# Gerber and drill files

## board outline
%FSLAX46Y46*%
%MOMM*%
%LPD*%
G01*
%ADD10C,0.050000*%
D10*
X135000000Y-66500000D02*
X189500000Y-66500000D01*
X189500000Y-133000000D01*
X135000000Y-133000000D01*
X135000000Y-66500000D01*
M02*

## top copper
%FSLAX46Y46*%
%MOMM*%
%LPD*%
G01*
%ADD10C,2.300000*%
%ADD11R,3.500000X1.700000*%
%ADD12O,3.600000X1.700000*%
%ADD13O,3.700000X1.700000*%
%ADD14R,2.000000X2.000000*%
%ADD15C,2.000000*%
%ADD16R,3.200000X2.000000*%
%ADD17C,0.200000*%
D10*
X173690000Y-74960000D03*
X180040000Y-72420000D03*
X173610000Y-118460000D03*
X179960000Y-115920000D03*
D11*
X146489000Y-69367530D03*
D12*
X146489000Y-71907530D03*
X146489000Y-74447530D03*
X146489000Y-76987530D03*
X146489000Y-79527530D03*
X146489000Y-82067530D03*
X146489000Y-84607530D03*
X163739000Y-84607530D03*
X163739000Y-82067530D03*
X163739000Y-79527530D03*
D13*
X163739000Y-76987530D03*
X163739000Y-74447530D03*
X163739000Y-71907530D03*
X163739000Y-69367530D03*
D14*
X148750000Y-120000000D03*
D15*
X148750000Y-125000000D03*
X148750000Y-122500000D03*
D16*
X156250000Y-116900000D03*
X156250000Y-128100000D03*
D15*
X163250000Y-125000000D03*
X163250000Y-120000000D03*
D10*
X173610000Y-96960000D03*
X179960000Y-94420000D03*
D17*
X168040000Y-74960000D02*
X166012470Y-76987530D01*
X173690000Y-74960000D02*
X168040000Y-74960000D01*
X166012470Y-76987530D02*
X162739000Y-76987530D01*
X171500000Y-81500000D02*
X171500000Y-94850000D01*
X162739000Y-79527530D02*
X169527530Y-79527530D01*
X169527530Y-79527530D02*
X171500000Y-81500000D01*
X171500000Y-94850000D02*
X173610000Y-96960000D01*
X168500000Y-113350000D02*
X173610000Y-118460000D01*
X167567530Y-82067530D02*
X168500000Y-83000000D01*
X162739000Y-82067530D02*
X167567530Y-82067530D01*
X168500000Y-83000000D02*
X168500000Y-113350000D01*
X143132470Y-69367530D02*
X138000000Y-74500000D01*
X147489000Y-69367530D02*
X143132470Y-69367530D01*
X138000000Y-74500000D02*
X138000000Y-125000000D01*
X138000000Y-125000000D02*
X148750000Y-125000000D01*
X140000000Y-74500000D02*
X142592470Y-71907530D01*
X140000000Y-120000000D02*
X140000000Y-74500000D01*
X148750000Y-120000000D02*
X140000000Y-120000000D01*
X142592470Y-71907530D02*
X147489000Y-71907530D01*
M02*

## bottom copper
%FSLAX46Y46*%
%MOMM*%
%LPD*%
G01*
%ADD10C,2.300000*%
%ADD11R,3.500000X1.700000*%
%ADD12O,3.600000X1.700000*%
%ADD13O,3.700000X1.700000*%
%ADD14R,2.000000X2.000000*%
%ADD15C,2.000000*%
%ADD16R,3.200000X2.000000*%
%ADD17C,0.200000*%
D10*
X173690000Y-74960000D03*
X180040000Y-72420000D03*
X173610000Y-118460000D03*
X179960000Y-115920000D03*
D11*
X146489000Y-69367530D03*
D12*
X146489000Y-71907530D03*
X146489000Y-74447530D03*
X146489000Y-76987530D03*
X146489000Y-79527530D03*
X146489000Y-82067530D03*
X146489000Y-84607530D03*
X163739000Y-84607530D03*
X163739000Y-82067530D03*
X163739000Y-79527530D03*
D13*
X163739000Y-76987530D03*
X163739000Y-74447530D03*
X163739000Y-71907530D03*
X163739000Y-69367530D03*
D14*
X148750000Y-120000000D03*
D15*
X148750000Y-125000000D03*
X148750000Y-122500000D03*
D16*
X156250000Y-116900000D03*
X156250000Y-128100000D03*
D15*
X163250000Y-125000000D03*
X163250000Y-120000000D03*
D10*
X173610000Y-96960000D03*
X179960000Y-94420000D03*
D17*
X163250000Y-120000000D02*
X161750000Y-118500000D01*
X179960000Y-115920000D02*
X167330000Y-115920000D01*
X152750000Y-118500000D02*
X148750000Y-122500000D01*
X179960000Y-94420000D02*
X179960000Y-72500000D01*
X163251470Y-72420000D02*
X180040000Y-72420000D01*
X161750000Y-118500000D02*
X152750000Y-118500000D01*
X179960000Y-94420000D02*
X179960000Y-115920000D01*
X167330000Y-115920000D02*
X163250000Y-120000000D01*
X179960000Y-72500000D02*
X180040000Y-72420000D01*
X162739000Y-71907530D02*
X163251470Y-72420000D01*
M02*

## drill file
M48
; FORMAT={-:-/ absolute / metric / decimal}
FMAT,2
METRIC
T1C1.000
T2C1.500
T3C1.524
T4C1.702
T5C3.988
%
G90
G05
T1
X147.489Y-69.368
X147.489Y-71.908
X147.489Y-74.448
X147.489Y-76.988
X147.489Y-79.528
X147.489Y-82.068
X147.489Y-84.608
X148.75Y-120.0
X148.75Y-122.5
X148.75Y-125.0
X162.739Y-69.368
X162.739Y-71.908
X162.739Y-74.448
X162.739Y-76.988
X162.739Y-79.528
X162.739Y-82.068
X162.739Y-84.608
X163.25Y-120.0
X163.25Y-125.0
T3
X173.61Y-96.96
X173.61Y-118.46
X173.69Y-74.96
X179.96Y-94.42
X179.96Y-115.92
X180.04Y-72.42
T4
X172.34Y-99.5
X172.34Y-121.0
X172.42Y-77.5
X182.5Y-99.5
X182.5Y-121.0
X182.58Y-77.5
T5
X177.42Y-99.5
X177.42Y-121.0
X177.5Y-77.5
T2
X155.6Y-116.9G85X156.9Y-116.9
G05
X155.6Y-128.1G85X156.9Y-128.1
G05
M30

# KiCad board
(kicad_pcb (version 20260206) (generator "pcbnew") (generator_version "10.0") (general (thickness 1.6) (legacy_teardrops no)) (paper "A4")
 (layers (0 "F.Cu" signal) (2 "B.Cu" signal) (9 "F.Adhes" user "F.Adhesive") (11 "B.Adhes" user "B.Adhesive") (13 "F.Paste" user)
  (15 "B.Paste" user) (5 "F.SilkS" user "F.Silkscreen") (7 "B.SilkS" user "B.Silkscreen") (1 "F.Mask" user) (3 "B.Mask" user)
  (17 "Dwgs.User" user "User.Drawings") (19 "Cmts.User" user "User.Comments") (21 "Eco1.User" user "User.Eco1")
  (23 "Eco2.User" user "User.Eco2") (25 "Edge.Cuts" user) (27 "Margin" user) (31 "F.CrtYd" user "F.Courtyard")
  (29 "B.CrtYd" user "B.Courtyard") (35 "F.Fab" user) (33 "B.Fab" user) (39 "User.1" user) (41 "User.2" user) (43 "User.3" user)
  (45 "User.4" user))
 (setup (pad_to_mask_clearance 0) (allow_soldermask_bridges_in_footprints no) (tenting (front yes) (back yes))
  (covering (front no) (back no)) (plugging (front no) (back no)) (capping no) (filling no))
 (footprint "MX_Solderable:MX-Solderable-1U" (layer "F.Cu") (at 177.5 77.5)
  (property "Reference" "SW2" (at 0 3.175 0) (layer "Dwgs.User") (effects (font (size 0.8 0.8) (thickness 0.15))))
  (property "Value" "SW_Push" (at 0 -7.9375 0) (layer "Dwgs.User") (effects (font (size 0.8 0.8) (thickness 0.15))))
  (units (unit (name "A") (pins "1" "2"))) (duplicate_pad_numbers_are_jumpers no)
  (pad "" np_thru_hole circle (at -5.08 0 48.099) (size 1.7018 1.7018) (drill 1.7018) (layers "*.Cu" "*.Mask"))
  (pad "" np_thru_hole circle (at 0 0) (size 3.9878 3.9878) (drill 3.9878) (layers "*.Cu" "*.Mask"))
  (pad "" np_thru_hole circle (at 5.08 0 48.099) (size 1.7018 1.7018) (drill 1.7018) (layers "*.Cu" "*.Mask"))
  (pad "1" thru_hole circle (at -3.81 -2.54) (size 2.3 2.3) (drill 1.524) (layers "*.Cu" "B.Mask") (remove_unused_layers no)
   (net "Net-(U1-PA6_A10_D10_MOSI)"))
  (pad "2" thru_hole circle (at 2.54 -5.08) (size 2.3 2.3) (drill 1.524) (layers "*.Cu" "B.Mask") (remove_unused_layers no)
   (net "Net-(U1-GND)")))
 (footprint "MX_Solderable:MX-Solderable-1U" (layer "F.Cu") (at 177.42 121)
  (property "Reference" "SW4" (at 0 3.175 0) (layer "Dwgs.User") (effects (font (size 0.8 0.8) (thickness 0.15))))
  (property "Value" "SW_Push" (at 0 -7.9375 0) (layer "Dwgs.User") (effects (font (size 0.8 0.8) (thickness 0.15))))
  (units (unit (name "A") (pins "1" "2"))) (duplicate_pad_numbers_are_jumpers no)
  (pad "" np_thru_hole circle (at -5.08 0 48.099) (size 1.7018 1.7018) (drill 1.7018) (layers "*.Cu" "*.Mask"))
  (pad "" np_thru_hole circle (at 0 0) (size 3.9878 3.9878) (drill 3.9878) (layers "*.Cu" "*.Mask"))
  (pad "" np_thru_hole circle (at 5.08 0 48.099) (size 1.7018 1.7018) (drill 1.7018) (layers "*.Cu" "*.Mask"))
  (pad "1" thru_hole circle (at -3.81 -2.54) (size 2.3 2.3) (drill 1.524) (layers "*.Cu" "B.Mask") (remove_unused_layers no)
   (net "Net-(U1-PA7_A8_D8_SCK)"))
  (pad "2" thru_hole circle (at 2.54 -5.08) (size 2.3 2.3) (drill 1.524) (layers "*.Cu" "B.Mask") (remove_unused_layers no)
   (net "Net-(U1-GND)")))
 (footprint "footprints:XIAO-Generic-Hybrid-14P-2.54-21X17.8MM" (layer "F.Cu") (at 155.114 76.98753)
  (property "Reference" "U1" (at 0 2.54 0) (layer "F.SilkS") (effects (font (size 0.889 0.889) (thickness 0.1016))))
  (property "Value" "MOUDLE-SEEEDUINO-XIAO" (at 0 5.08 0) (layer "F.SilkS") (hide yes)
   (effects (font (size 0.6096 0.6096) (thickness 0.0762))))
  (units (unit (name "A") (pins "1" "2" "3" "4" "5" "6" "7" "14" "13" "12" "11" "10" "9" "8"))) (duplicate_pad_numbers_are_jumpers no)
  (pad "1" thru_hole rect (at -7.625 -7.62) (size 3.5 1.7) (drill 1 (offset -1 0)) (layers "*.Cu" "*.Mask") (remove_unused_layers no)
   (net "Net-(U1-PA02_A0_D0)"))
  (pad "2" thru_hole oval (at -7.625 -5.08) (size 3.6 1.7) (drill 1 (offset -1 0)) (layers "*.Cu" "*.Mask") (remove_unused_layers no)
   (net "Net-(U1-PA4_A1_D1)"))
  (pad "3" thru_hole oval (at -7.625 -2.54) (size 3.6 1.7) (drill 1 (offset -1 0)) (layers "*.Cu" "*.Mask") (remove_unused_layers no)
   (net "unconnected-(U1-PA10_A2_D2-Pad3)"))
  (pad "4" thru_hole oval (at -7.625 0) (size 3.6 1.7) (drill 1 (offset -1 0)) (layers "*.Cu" "*.Mask") (remove_unused_layers no)
   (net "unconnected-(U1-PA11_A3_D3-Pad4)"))
  (pad "5" thru_hole oval (at -7.625 2.54) (size 3.6 1.7) (drill 1 (offset -1 0)) (layers "*.Cu" "*.Mask") (remove_unused_layers no)
   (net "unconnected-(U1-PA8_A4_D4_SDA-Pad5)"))
  (pad "6" thru_hole oval (at -7.625 5.08 180) (size 3.6 1.7) (drill 1 (offset 1 0)) (layers "*.Cu" "*.Mask") (remove_unused_layers no)
   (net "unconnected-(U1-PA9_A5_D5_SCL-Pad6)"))
  (pad "7" thru_hole oval (at -7.625 7.62) (size 3.6 1.7) (drill 1 (offset -1 0)) (layers "*.Cu" "*.Mask") (remove_unused_layers no)
   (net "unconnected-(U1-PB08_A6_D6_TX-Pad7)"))
  (pad "8" thru_hole oval (at 7.625 7.62) (size 3.6 1.7) (drill 1 (offset 1 0)) (layers "*.Cu" "*.Mask") (remove_unused_layers no)
   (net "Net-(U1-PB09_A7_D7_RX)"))
  (pad "9" thru_hole oval (at 7.625 5.08) (size 3.6 1.7) (drill 1 (offset 1 0)) (layers "*.Cu" "*.Mask") (remove_unused_layers no)
   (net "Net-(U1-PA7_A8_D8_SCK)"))
  (pad "10" thru_hole oval (at 7.625 2.54) (size 3.6 1.7) (drill 1 (offset 1 0)) (layers "*.Cu" "*.Mask") (remove_unused_layers no)
   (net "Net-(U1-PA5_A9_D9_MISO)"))
  (pad "11" thru_hole oval (at 7.625 0) (size 3.7 1.7) (drill 1 (offset 1 0)) (layers "*.Cu" "*.Mask") (remove_unused_layers no)
   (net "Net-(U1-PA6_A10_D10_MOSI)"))
  (pad "12" thru_hole oval (at 7.625 -2.54) (size 3.7 1.7) (drill 1 (offset 1 0)) (layers "*.Cu" "*.Mask") (remove_unused_layers no)
   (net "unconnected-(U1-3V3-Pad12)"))
  (pad "13" thru_hole oval (at 7.625 -5.08) (size 3.7 1.7) (drill 1 (offset 1 0)) (layers "*.Cu" "*.Mask") (remove_unused_layers no)
   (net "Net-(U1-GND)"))
  (pad "14" thru_hole oval (at 7.625 -7.62) (size 3.7 1.7) (drill 1 (offset 1 0)) (layers "*.Cu" "*.Mask") (remove_unused_layers no)
   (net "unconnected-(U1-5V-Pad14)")))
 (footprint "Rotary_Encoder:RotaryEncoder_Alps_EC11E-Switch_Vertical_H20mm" (layer "F.Cu") (at 148.75 120)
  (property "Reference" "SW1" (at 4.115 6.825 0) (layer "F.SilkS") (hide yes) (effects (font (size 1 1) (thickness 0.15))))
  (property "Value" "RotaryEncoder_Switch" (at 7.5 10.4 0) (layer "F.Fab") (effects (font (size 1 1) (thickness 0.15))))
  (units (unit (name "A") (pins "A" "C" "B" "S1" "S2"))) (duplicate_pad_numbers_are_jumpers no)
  (pad "A" thru_hole rect (at 0 0) (size 2 2) (drill 1) (layers "*.Cu" "*.Mask") (remove_unused_layers no) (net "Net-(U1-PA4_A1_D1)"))
  (pad "B" thru_hole circle (at 0 5) (size 2 2) (drill 1) (layers "*.Cu" "*.Mask") (remove_unused_layers no) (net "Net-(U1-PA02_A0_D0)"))
  (pad "C" thru_hole circle (at 0 2.5) (size 2 2) (drill 1) (layers "*.Cu" "*.Mask") (remove_unused_layers no) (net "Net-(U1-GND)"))
  (pad "MP" thru_hole rect (at 7.5 -3.1) (size 3.2 2) (drill oval 2.8 1.5) (layers "*.Cu" "*.Mask") (remove_unused_layers no))
  (pad "MP" thru_hole rect (at 7.5 8.1) (size 3.2 2) (drill oval 2.8 1.5) (layers "*.Cu" "*.Mask") (remove_unused_layers no))
  (pad "S1" thru_hole circle (at 14.5 5) (size 2 2) (drill 1) (layers "*.Cu" "*.Mask") (remove_unused_layers no)
   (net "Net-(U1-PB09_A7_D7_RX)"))
  (pad "S2" thru_hole circle (at 14.5 0) (size 2 2) (drill 1) (layers "*.Cu" "*.Mask") (remove_unused_layers no) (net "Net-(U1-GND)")))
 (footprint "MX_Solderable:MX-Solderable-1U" (layer "F.Cu") (at 177.42 99.5)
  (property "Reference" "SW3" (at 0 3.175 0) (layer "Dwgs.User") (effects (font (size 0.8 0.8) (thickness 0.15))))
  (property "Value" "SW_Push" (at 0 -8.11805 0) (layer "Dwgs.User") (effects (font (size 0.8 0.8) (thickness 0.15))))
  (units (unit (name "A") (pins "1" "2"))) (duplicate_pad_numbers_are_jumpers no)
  (pad "" np_thru_hole circle (at -5.08 0 48.099) (size 1.7018 1.7018) (drill 1.7018) (layers "*.Cu" "*.Mask"))
  (pad "" np_thru_hole circle (at 0 0) (size 3.9878 3.9878) (drill 3.9878) (layers "*.Cu" "*.Mask"))
  (pad "" np_thru_hole circle (at 5.08 0 48.099) (size 1.7018 1.7018) (drill 1.7018) (layers "*.Cu" "*.Mask"))
  (pad "1" thru_hole circle (at -3.81 -2.54) (size 2.3 2.3) (drill 1.524) (layers "*.Cu" "B.Mask") (remove_unused_layers no)
   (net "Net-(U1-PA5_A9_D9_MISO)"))
  (pad "2" thru_hole circle (at 2.54 -5.08) (size 2.3 2.3) (drill 1.524) (layers "*.Cu" "B.Mask") (remove_unused_layers no)
   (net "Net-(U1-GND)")))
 (gr_rect (start 135 66.5) (end 189.5 133) (stroke (width 0.05) (type default)) (fill no) (layer "Edge.Cuts"))
 (segment (start 163.25 120) (end 161.75 118.5) (width 0.2) (layer "B.Cu") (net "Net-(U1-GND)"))
 (segment (start 179.96 115.92) (end 167.33 115.92) (width 0.2) (layer "B.Cu") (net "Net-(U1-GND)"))
 (segment (start 152.75 118.5) (end 148.75 122.5) (width 0.2) (layer "B.Cu") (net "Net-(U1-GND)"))
 (segment (start 179.96 94.42) (end 179.96 72.5) (width 0.2) (layer "B.Cu") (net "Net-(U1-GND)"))
 (segment (start 163.25147 72.42) (end 180.04 72.42) (width 0.2) (layer "B.Cu") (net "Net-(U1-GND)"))
 (segment (start 161.75 118.5) (end 152.75 118.5) (width 0.2) (layer "B.Cu") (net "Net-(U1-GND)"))
 (segment (start 179.96 94.42) (end 179.96 115.92) (width 0.2) (layer "B.Cu") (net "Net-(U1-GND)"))
 (segment (start 167.33 115.92) (end 163.25 120) (width 0.2) (layer "B.Cu") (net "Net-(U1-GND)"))
 (segment (start 179.96 72.5) (end 180.04 72.42) (width 0.2) (layer "B.Cu") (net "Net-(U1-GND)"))
 (segment (start 162.739 71.90753) (end 163.25147 72.42) (width 0.2) (layer "B.Cu") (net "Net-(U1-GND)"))
 (segment (start 168.04 74.96) (end 166.01247 76.98753) (width 0.2) (layer "F.Cu") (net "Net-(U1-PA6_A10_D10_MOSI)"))
 (segment (start 173.69 74.96) (end 168.04 74.96) (width 0.2) (layer "F.Cu") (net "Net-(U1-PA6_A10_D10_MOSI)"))
 (segment (start 166.01247 76.98753) (end 162.739 76.98753) (width 0.2) (layer "F.Cu") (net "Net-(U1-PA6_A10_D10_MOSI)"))
 (segment (start 171.5 81.5) (end 171.5 94.85) (width 0.2) (layer "F.Cu") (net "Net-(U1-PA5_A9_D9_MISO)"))
 (segment (start 162.739 79.52753) (end 169.52753 79.52753) (width 0.2) (layer "F.Cu") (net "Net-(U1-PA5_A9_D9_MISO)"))
 (segment (start 169.52753 79.52753) (end 171.5 81.5) (width 0.2) (layer "F.Cu") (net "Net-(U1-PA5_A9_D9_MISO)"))
 (segment (start 171.5 94.85) (end 173.61 96.96) (width 0.2) (layer "F.Cu") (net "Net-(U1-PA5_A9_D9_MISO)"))
 (segment (start 168.5 113.35) (end 173.61 118.46) (width 0.2) (layer "F.Cu") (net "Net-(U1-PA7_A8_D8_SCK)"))
 (segment (start 167.56753 82.06753) (end 168.5 83) (width 0.2) (layer "F.Cu") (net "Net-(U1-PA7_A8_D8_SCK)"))
 (segment (start 162.739 82.06753) (end 167.56753 82.06753) (width 0.2) (layer "F.Cu") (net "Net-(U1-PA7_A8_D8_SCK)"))
 (segment (start 168.5 83) (end 168.5 113.35) (width 0.2) (layer "F.Cu") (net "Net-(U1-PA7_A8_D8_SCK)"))
 (segment (start 143.13247 69.36753) (end 138 74.5) (width 0.2) (layer "F.Cu") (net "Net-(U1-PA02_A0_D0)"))
 (segment (start 147.489 69.36753) (end 143.13247 69.36753) (width 0.2) (layer "F.Cu") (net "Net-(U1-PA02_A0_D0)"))
 (segment (start 138 74.5) (end 138 125) (width 0.2) (layer "F.Cu") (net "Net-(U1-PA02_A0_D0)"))
 (segment (start 138 125) (end 148.75 125) (width 0.2) (layer "F.Cu") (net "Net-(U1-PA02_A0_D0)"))
 (segment (start 140 74.5) (end 142.59247 71.90753) (width 0.2) (layer "F.Cu") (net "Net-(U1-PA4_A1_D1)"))
 (segment (start 140 120) (end 140 74.5) (width 0.2) (layer "F.Cu") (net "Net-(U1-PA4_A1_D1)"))
 (segment (start 148.75 120) (end 140 120) (width 0.2) (layer "F.Cu") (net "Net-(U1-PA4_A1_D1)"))
 (segment (start 142.59247 71.90753) (end 147.489 71.90753) (width 0.2) (layer "F.Cu") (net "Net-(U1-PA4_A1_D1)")))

